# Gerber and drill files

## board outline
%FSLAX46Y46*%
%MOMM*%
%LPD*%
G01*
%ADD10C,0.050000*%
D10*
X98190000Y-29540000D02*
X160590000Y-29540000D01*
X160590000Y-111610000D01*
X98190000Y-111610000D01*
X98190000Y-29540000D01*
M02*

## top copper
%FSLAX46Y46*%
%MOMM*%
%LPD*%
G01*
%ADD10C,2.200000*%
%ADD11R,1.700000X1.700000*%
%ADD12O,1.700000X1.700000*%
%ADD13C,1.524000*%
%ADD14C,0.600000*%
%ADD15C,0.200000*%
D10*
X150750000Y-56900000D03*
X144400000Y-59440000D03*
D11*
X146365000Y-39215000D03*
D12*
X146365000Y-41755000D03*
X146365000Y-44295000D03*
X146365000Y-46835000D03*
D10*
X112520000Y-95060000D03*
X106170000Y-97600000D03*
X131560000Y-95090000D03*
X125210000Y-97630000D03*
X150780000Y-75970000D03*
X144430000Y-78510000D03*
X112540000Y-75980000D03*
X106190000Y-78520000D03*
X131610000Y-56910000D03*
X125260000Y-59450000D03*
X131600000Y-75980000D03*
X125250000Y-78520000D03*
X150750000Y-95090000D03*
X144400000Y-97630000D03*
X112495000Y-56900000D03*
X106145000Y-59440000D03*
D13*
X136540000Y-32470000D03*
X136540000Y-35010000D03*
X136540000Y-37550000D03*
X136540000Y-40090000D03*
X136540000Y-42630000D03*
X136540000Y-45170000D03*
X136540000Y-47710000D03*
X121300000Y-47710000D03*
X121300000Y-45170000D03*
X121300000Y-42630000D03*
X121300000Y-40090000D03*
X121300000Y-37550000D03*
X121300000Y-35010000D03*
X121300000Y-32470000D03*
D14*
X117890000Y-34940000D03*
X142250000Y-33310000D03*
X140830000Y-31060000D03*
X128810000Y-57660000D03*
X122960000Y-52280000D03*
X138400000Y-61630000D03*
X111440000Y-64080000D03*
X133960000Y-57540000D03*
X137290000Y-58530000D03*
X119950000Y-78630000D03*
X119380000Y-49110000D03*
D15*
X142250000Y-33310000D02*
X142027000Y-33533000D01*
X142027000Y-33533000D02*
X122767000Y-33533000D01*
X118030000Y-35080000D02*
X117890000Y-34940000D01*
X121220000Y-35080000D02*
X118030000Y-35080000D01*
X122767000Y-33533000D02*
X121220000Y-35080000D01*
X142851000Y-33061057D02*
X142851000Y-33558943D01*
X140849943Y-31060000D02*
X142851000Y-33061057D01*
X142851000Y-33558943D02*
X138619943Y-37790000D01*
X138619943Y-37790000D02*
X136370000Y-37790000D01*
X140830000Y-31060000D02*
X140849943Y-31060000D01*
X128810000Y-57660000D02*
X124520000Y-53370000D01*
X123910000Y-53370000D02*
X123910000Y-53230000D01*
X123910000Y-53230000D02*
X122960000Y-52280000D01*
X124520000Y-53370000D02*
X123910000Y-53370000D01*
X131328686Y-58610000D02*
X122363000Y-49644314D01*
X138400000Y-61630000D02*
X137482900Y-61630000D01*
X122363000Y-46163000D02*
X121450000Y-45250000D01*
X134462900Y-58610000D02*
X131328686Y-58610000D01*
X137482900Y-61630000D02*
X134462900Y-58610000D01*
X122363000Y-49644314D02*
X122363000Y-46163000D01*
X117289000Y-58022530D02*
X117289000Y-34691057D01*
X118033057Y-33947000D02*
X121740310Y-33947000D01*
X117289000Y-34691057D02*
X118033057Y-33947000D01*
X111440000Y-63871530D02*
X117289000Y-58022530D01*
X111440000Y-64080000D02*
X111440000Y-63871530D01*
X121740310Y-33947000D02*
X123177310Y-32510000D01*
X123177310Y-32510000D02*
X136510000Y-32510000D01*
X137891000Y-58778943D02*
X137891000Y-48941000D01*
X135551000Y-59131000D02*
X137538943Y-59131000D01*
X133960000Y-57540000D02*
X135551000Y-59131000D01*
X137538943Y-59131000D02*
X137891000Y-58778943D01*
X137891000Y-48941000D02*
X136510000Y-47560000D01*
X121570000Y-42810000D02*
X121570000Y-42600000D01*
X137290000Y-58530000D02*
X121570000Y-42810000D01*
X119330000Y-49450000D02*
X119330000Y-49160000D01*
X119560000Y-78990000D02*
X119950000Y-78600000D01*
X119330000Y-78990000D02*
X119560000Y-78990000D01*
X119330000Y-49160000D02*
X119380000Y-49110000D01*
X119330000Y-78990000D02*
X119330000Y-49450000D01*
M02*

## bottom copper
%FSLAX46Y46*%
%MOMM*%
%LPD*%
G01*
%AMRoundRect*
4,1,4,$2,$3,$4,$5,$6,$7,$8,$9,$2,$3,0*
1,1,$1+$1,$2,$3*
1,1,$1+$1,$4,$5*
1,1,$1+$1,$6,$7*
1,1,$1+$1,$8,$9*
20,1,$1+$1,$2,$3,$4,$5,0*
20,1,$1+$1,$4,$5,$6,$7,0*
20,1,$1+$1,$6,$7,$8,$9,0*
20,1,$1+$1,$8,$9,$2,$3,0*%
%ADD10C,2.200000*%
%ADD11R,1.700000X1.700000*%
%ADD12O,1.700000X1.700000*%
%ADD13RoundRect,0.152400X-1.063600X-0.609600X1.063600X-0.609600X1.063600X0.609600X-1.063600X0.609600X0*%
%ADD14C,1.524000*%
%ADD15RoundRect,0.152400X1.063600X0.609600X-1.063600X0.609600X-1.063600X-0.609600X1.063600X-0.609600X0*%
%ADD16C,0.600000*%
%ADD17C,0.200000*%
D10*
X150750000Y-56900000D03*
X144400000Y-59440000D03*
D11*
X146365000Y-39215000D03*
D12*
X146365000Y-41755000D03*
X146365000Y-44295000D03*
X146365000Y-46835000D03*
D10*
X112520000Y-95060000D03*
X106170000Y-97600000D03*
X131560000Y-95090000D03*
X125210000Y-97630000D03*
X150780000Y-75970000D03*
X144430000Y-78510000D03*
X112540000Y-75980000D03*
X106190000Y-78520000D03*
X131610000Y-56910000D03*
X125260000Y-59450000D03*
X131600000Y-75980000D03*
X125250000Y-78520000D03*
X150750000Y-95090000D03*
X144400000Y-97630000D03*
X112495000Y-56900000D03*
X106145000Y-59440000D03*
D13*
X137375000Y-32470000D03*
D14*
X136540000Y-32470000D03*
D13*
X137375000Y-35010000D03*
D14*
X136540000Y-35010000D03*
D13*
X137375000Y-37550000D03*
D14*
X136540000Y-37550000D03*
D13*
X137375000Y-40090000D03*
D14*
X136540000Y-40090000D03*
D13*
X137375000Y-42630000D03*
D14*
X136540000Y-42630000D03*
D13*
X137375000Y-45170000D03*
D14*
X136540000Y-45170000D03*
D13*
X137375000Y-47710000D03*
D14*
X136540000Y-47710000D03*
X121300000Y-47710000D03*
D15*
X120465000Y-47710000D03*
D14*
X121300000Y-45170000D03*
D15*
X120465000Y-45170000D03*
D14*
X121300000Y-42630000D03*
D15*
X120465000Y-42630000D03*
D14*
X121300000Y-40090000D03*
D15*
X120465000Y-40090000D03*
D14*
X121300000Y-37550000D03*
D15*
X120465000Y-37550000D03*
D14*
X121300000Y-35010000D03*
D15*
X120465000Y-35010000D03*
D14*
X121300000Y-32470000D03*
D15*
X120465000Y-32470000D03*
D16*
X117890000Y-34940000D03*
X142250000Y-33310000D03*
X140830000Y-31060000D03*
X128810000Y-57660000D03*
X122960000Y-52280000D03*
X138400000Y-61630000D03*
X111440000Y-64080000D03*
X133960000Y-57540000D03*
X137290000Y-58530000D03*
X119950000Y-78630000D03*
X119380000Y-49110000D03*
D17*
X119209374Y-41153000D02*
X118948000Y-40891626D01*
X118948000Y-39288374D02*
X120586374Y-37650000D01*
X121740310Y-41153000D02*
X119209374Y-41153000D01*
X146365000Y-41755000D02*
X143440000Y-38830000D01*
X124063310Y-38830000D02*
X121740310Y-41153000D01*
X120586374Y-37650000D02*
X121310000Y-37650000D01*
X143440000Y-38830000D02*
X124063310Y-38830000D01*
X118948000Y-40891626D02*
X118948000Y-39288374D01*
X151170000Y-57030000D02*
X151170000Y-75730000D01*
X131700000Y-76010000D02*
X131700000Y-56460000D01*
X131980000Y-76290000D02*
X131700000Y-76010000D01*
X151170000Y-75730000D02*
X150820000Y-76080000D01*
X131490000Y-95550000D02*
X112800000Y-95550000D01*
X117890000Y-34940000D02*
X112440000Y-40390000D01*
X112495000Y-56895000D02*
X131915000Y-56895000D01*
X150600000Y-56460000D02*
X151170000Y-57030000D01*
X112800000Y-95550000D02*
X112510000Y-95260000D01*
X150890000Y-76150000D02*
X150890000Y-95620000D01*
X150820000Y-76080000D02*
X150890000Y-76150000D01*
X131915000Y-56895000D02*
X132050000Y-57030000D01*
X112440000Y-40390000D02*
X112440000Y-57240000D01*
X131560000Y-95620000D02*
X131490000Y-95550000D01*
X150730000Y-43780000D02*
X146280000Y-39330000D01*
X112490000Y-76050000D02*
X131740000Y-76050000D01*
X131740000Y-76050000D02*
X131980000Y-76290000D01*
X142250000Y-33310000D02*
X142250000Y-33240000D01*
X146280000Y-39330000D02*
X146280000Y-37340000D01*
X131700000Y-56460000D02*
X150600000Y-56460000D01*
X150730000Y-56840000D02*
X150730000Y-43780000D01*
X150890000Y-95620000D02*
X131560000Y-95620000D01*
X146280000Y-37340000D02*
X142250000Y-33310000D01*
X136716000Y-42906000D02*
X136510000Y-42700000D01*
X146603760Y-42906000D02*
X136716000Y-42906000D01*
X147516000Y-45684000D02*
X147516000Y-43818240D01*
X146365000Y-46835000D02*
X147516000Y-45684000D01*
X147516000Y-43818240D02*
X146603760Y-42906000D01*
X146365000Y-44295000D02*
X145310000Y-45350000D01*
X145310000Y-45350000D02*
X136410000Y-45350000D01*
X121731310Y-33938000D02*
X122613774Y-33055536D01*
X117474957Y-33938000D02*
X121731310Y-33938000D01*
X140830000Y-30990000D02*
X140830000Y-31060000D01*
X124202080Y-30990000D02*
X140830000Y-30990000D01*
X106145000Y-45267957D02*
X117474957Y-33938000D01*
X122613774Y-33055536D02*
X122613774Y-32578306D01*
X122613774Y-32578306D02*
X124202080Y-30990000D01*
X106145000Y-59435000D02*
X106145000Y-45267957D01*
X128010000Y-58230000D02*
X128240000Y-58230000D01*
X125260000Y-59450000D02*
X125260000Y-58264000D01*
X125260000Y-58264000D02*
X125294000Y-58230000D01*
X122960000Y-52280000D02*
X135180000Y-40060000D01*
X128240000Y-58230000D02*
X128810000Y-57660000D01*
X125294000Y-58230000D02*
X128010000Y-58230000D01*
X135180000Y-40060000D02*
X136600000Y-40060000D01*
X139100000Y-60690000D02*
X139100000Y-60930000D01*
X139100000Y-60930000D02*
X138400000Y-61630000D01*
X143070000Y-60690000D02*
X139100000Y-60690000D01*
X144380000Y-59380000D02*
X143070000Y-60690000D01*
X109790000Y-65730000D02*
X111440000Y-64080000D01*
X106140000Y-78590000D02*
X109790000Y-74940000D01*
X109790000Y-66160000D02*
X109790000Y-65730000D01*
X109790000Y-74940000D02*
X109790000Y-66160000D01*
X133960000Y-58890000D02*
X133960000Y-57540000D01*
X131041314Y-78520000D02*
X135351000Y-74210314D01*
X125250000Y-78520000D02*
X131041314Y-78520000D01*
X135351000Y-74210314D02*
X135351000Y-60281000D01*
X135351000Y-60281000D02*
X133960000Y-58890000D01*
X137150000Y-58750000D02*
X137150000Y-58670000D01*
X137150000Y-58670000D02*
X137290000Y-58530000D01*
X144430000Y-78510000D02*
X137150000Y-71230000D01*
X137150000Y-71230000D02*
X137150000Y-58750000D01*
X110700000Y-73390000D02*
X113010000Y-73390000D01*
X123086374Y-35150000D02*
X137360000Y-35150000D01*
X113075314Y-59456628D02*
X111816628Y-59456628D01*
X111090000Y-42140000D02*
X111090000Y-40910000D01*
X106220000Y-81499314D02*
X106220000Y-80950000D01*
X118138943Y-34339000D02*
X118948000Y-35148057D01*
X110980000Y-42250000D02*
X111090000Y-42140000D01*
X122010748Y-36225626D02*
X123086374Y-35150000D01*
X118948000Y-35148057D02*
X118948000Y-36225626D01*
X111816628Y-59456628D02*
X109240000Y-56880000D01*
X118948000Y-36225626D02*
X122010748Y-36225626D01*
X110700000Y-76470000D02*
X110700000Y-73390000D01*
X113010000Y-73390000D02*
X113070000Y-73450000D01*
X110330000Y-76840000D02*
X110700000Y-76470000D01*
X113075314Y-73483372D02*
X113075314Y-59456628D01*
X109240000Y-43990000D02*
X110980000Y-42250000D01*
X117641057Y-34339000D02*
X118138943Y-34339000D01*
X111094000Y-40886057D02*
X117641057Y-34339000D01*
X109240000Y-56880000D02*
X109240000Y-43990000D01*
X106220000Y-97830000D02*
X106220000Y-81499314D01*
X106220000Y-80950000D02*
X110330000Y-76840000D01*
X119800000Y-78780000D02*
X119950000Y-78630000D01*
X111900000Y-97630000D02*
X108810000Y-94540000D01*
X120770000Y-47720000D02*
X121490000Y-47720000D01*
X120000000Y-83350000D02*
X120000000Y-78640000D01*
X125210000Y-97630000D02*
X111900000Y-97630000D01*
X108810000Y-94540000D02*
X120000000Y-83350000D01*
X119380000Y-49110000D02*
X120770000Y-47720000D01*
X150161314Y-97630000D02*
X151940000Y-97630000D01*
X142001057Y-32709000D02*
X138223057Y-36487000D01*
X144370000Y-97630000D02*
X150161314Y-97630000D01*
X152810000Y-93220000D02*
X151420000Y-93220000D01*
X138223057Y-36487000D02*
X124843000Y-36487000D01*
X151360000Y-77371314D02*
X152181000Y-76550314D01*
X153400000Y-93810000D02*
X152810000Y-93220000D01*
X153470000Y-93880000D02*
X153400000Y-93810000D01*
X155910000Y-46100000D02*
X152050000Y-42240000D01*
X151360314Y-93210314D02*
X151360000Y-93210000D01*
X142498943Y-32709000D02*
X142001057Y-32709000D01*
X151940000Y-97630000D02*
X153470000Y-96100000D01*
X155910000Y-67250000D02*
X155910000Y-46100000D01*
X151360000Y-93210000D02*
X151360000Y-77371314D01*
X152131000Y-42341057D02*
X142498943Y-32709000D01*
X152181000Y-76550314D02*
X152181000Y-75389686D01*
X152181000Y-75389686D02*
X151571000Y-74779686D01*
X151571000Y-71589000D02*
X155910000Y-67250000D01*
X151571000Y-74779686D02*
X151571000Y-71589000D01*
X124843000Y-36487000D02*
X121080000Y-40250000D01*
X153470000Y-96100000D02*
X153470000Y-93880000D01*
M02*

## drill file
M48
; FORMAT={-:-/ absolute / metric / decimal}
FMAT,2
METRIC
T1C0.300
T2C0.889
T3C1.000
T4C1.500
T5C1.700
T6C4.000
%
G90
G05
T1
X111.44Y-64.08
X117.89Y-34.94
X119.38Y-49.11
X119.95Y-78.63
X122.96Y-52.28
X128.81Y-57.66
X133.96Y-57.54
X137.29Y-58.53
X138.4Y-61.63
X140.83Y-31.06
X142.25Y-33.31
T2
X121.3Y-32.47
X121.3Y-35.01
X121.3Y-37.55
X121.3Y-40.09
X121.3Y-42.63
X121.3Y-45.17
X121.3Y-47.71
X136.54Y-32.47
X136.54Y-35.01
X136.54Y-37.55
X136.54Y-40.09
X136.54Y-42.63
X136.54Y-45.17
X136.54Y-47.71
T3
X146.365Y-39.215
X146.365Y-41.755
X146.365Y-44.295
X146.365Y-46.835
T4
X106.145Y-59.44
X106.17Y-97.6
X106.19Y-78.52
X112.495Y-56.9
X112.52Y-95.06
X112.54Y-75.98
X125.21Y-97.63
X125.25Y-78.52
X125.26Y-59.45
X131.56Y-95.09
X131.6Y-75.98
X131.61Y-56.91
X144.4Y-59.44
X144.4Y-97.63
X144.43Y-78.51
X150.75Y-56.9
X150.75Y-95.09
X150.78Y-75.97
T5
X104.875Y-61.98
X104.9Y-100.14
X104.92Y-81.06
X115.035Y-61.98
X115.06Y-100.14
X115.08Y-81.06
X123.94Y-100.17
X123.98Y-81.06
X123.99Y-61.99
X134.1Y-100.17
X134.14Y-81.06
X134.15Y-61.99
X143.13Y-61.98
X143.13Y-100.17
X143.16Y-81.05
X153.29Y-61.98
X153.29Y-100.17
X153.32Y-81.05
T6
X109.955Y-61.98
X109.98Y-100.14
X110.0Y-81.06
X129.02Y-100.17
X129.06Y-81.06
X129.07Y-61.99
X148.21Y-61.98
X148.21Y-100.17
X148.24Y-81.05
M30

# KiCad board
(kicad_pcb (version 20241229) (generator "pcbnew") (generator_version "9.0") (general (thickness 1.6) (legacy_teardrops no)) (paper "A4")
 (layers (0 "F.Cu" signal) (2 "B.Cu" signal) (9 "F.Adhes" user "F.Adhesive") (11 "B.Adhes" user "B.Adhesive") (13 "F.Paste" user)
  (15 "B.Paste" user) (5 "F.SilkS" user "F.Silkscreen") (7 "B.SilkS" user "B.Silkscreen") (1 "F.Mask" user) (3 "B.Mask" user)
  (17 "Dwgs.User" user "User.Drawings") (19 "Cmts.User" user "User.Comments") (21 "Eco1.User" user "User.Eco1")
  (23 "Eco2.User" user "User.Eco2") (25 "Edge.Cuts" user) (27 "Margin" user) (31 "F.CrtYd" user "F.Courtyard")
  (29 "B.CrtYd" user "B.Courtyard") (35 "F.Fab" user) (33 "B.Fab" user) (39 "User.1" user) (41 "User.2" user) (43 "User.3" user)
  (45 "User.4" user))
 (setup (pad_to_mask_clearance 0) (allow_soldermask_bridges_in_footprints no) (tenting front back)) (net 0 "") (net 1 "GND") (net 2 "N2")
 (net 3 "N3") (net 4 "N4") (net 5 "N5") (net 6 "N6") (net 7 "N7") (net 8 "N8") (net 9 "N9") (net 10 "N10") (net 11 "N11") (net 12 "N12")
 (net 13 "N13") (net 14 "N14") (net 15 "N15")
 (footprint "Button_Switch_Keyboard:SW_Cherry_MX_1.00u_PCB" (layer "F.Cu") (at 150.75 56.9)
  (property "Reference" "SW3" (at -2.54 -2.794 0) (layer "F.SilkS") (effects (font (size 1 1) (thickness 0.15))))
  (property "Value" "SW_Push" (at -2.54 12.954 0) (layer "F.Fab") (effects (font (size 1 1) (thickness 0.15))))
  (pad "" np_thru_hole circle (at -7.62 5.08) (size 1.7 1.7) (drill 1.7) (layers "*.Cu" "*.Mask"))
  (pad "" np_thru_hole circle (at -2.54 5.08) (size 4 4) (drill 4) (layers "*.Cu" "*.Mask"))
  (pad "" np_thru_hole circle (at 2.54 5.08) (size 1.7 1.7) (drill 1.7) (layers "*.Cu" "*.Mask"))
  (pad "1" thru_hole circle (at 0 0) (size 2.2 2.2) (drill 1.5) (layers "*.Cu" "*.Mask") (remove_unused_layers no) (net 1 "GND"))
  (pad "2" thru_hole circle (at -6.35 2.54) (size 2.2 2.2) (drill 1.5) (layers "*.Cu" "*.Mask") (remove_unused_layers no) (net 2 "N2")))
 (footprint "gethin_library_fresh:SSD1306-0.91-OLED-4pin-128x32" (layer "F.Cu") (at 109.865 37.025)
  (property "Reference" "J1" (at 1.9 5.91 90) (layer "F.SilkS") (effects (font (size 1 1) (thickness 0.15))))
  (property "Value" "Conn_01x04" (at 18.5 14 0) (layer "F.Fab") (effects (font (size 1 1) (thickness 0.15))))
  (pad "1" thru_hole rect (at 36.5 2.19) (size 1.7 1.7) (drill 1) (layers "*.Cu" "*.Mask") (remove_unused_layers no) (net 1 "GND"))
  (pad "2" thru_hole oval (at 36.5 4.73) (size 1.7 1.7) (drill 1) (layers "*.Cu" "*.Mask") (remove_unused_layers no) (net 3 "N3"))
  (pad "3" thru_hole oval (at 36.5 7.27) (size 1.7 1.7) (drill 1) (layers "*.Cu" "*.Mask") (remove_unused_layers no) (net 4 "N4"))
  (pad "4" thru_hole oval (at 36.5 9.81) (size 1.7 1.7) (drill 1) (layers "*.Cu" "*.Mask") (remove_unused_layers no) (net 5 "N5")))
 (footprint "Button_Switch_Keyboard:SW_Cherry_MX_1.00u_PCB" (layer "F.Cu") (at 112.52 95.06)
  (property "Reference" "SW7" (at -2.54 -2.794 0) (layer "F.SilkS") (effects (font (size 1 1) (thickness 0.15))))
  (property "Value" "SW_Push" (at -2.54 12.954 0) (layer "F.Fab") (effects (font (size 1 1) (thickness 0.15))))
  (pad "" np_thru_hole circle (at -7.62 5.08) (size 1.7 1.7) (drill 1.7) (layers "*.Cu" "*.Mask"))
  (pad "" np_thru_hole circle (at -2.54 5.08) (size 4 4) (drill 4) (layers "*.Cu" "*.Mask"))
  (pad "" np_thru_hole circle (at 2.54 5.08) (size 1.7 1.7) (drill 1.7) (layers "*.Cu" "*.Mask"))
  (pad "1" thru_hole circle (at 0 0) (size 2.2 2.2) (drill 1.5) (layers "*.Cu" "*.Mask") (remove_unused_layers no) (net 1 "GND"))
  (pad "2" thru_hole circle (at -6.35 2.54) (size 2.2 2.2) (drill 1.5) (layers "*.Cu" "*.Mask") (remove_unused_layers no) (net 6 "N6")))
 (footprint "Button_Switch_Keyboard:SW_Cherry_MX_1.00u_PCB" (layer "F.Cu") (at 131.56 95.09)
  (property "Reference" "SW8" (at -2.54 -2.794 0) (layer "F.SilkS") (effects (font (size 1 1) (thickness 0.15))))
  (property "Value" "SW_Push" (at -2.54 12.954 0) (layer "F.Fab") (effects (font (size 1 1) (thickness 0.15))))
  (pad "" np_thru_hole circle (at -7.62 5.08) (size 1.7 1.7) (drill 1.7) (layers "*.Cu" "*.Mask"))
  (pad "" np_thru_hole circle (at -2.54 5.08) (size 4 4) (drill 4) (layers "*.Cu" "*.Mask"))
  (pad "" np_thru_hole circle (at 2.54 5.08) (size 1.7 1.7) (drill 1.7) (layers "*.Cu" "*.Mask"))
  (pad "1" thru_hole circle (at 0 0) (size 2.2 2.2) (drill 1.5) (layers "*.Cu" "*.Mask") (remove_unused_layers no) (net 1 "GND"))
  (pad "2" thru_hole circle (at -6.35 2.54) (size 2.2 2.2) (drill 1.5) (layers "*.Cu" "*.Mask") (remove_unused_layers no) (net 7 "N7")))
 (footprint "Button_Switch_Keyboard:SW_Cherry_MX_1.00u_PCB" (layer "F.Cu") (at 150.78 75.97)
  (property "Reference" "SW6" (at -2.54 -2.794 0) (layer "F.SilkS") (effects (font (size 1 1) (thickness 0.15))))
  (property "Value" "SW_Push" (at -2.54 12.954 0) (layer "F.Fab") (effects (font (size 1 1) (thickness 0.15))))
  (pad "" np_thru_hole circle (at -7.62 5.08) (size 1.7 1.7) (drill 1.7) (layers "*.Cu" "*.Mask"))
  (pad "" np_thru_hole circle (at -2.54 5.08) (size 4 4) (drill 4) (layers "*.Cu" "*.Mask"))
  (pad "" np_thru_hole circle (at 2.54 5.08) (size 1.7 1.7) (drill 1.7) (layers "*.Cu" "*.Mask"))
  (pad "1" thru_hole circle (at 0 0) (size 2.2 2.2) (drill 1.5) (layers "*.Cu" "*.Mask") (remove_unused_layers no) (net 1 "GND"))
  (pad "2" thru_hole circle (at -6.35 2.54) (size 2.2 2.2) (drill 1.5) (layers "*.Cu" "*.Mask") (remove_unused_layers no) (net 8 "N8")))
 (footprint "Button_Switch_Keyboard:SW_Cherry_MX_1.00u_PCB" (layer "F.Cu") (at 112.54 75.98)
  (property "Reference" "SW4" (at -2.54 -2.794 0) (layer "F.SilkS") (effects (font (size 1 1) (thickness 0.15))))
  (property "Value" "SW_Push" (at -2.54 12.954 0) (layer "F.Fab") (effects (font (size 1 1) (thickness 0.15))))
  (pad "" np_thru_hole circle (at -7.62 5.08) (size 1.7 1.7) (drill 1.7) (layers "*.Cu" "*.Mask"))
  (pad "" np_thru_hole circle (at -2.54 5.08) (size 4 4) (drill 4) (layers "*.Cu" "*.Mask"))
  (pad "" np_thru_hole circle (at 2.54 5.08) (size 1.7 1.7) (drill 1.7) (layers "*.Cu" "*.Mask"))
  (pad "1" thru_hole circle (at 0 0) (size 2.2 2.2) (drill 1.5) (layers "*.Cu" "*.Mask") (remove_unused_layers no) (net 1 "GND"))
  (pad "2" thru_hole circle (at -6.35 2.54) (size 2.2 2.2) (drill 1.5) (layers "*.Cu" "*.Mask") (remove_unused_layers no) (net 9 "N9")))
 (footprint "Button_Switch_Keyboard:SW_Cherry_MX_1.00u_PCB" (layer "F.Cu") (at 131.61 56.91)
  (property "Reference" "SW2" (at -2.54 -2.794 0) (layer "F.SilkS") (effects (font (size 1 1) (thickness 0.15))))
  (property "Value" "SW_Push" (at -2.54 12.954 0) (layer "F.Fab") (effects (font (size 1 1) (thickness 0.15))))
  (pad "" np_thru_hole circle (at -7.62 5.08) (size 1.7 1.7) (drill 1.7) (layers "*.Cu" "*.Mask"))
  (pad "" np_thru_hole circle (at -2.54 5.08) (size 4 4) (drill 4) (layers "*.Cu" "*.Mask"))
  (pad "" np_thru_hole circle (at 2.54 5.08) (size 1.7 1.7) (drill 1.7) (layers "*.Cu" "*.Mask"))
  (pad "1" thru_hole circle (at 0 0) (size 2.2 2.2) (drill 1.5) (layers "*.Cu" "*.Mask") (remove_unused_layers no) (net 1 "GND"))
  (pad "2" thru_hole circle (at -6.35 2.54) (size 2.2 2.2) (drill 1.5) (layers "*.Cu" "*.Mask") (remove_unused_layers no) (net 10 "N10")))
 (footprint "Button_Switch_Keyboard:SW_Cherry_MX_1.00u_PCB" (layer "F.Cu") (at 131.6 75.98)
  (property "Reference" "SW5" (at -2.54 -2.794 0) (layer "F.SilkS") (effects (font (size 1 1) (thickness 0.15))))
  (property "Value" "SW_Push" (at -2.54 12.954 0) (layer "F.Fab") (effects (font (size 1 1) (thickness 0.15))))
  (pad "" np_thru_hole circle (at -7.62 5.08) (size 1.7 1.7) (drill 1.7) (layers "*.Cu" "*.Mask"))
  (pad "" np_thru_hole circle (at -2.54 5.08) (size 4 4) (drill 4) (layers "*.Cu" "*.Mask"))
  (pad "" np_thru_hole circle (at 2.54 5.08) (size 1.7 1.7) (drill 1.7) (layers "*.Cu" "*.Mask"))
  (pad "1" thru_hole circle (at 0 0) (size 2.2 2.2) (drill 1.5) (layers "*.Cu" "*.Mask") (remove_unused_layers no) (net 1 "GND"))
  (pad "2" thru_hole circle (at -6.35 2.54) (size 2.2 2.2) (drill 1.5) (layers "*.Cu" "*.Mask") (remove_unused_layers no) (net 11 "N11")))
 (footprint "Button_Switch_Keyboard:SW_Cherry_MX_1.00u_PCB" (layer "F.Cu") (at 150.75 95.09)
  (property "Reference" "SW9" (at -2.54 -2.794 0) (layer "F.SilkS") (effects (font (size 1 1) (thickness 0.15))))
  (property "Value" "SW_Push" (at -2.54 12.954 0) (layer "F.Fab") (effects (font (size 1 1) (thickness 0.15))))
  (pad "" np_thru_hole circle (at -7.62 5.08) (size 1.7 1.7) (drill 1.7) (layers "*.Cu" "*.Mask"))
  (pad "" np_thru_hole circle (at -2.54 5.08) (size 4 4) (drill 4) (layers "*.Cu" "*.Mask"))
  (pad "" np_thru_hole circle (at 2.54 5.08) (size 1.7 1.7) (drill 1.7) (layers "*.Cu" "*.Mask"))
  (pad "1" thru_hole circle (at 0 0) (size 2.2 2.2) (drill 1.5) (layers "*.Cu" "*.Mask") (remove_unused_layers no) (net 1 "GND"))
  (pad "2" thru_hole circle (at -6.35 2.54) (size 2.2 2.2) (drill 1.5) (layers "*.Cu" "*.Mask") (remove_unused_layers no) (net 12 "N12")))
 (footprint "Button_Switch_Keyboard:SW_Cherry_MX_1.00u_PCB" (layer "F.Cu") (at 112.495 56.9)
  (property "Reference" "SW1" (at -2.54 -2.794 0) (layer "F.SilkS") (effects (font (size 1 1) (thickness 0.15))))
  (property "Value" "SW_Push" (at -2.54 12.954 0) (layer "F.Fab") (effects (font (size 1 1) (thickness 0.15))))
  (pad "" np_thru_hole circle (at -7.62 5.08) (size 1.7 1.7) (drill 1.7) (layers "*.Cu" "*.Mask"))
  (pad "" np_thru_hole circle (at -2.54 5.08) (size 4 4) (drill 4) (layers "*.Cu" "*.Mask"))
  (pad "" np_thru_hole circle (at 2.54 5.08) (size 1.7 1.7) (drill 1.7) (layers "*.Cu" "*.Mask"))
  (pad "1" thru_hole circle (at 0 0) (size 2.2 2.2) (drill 1.5) (layers "*.Cu" "*.Mask") (remove_unused_layers no) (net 1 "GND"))
  (pad "2" thru_hole circle (at -6.35 2.54) (size 2.2 2.2) (drill 1.5) (layers "*.Cu" "*.Mask") (remove_unused_layers no) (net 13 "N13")))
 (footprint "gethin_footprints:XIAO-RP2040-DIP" (layer "B.Cu") (at 128.92 40.09 180)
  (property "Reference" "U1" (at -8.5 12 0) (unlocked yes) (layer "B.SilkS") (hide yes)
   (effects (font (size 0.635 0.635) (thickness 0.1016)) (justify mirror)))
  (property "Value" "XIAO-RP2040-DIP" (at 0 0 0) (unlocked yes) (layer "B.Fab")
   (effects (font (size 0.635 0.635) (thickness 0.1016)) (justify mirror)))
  (pad "1" smd roundrect (at -8.455 7.62) (size 2.432 1.524) (layers "B.Cu" "B.Mask") (roundrect_rratio 0.1) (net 9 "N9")
   (thermal_bridge_angle 45))
  (pad "1" thru_hole circle (at -7.62 7.62) (size 1.524 1.524) (drill 0.889) (layers "*.Cu" "*.Mask") (remove_unused_layers no) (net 9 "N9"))
  (pad "2" smd roundrect (at -8.455 5.08) (size 2.432 1.524) (layers "B.Cu" "B.Mask") (roundrect_rratio 0.1) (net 6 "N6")
   (thermal_bridge_angle 45))
  (pad "2" thru_hole circle (at -7.62 5.08) (size 1.524 1.524) (drill 0.889) (layers "*.Cu" "*.Mask") (remove_unused_layers no) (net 6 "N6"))
  (pad "3" smd roundrect (at -8.455 2.54) (size 2.432 1.524) (layers "B.Cu" "B.Mask") (roundrect_rratio 0.1) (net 13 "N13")
   (thermal_bridge_angle 45))
  (pad "3" thru_hole circle (at -7.62 2.54) (size 1.524 1.524) (drill 0.889) (layers "*.Cu" "*.Mask") (remove_unused_layers no)
   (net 13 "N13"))
  (pad "4" smd roundrect (at -8.455 0) (size 2.432 1.524) (layers "B.Cu" "B.Mask") (roundrect_rratio 0.1) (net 10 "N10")
   (thermal_bridge_angle 45))
  (pad "4" thru_hole circle (at -7.62 0) (size 1.524 1.524) (drill 0.889) (layers "*.Cu" "*.Mask") (remove_unused_layers no) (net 10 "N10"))
  (pad "5" smd roundrect (at -8.455 -2.54) (size 2.432 1.524) (layers "B.Cu" "B.Mask") (roundrect_rratio 0.1) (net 5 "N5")
   (thermal_bridge_angle 45))
  (pad "5" thru_hole circle (at -7.62 -2.54) (size 1.524 1.524) (drill 0.889) (layers "*.Cu" "*.Mask") (remove_unused_layers no)
   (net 5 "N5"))
  (pad "6" smd roundrect (at -8.455 -5.08) (size 2.432 1.524) (layers "B.Cu" "B.Mask") (roundrect_rratio 0.1) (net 4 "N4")
   (thermal_bridge_angle 45))
  (pad "6" thru_hole circle (at -7.62 -5.08) (size 1.524 1.524) (drill 0.889) (layers "*.Cu" "*.Mask") (remove_unused_layers no)
   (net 4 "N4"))
  (pad "7" smd roundrect (at -8.455 -7.62) (size 2.432 1.524) (layers "B.Cu" "B.Mask") (roundrect_rratio 0.1) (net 11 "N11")
   (thermal_bridge_angle 45))
  (pad "7" thru_hole circle (at -7.62 -7.62) (size 1.524 1.524) (drill 0.889) (layers "*.Cu" "*.Mask") (remove_unused_layers no)
   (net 11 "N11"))
  (pad "8" thru_hole circle (at 7.62 -7.62 180) (size 1.524 1.524) (drill 0.889) (layers "*.Cu" "*.Mask") (remove_unused_layers no)
   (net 7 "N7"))
  (pad "8" smd roundrect (at 8.455 -7.62 180) (size 2.432 1.524) (layers "B.Cu" "B.Mask") (roundrect_rratio 0.1) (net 7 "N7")
   (thermal_bridge_angle 45))
  (pad "9" thru_hole circle (at 7.62 -5.08 180) (size 1.524 1.524) (drill 0.889) (layers "*.Cu" "*.Mask") (remove_unused_layers no)
   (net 2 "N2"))
  (pad "9" smd roundrect (at 8.455 -5.08 180) (size 2.432 1.524) (layers "B.Cu" "B.Mask") (roundrect_rratio 0.1) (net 2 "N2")
   (thermal_bridge_angle 45))
  (pad "10" thru_hole circle (at 7.62 -2.54 180) (size 1.524 1.524) (drill 0.889) (layers "*.Cu" "*.Mask") (remove_unused_layers no)
   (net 8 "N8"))
  (pad "10" smd roundrect (at 8.455 -2.54 180) (size 2.432 1.524) (layers "B.Cu" "B.Mask") (roundrect_rratio 0.1) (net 8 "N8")
   (thermal_bridge_angle 45))
  (pad "11" thru_hole circle (at 7.62 0 180) (size 1.524 1.524) (drill 0.889) (layers "*.Cu" "*.Mask") (remove_unused_layers no)
   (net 12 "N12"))
  (pad "11" smd roundrect (at 8.455 0 180) (size 2.432 1.524) (layers "B.Cu" "B.Mask") (roundrect_rratio 0.1) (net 12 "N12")
   (thermal_bridge_angle 45))
  (pad "12" thru_hole circle (at 7.62 2.54 180) (size 1.524 1.524) (drill 0.889) (layers "*.Cu" "*.Mask") (remove_unused_layers no)
   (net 3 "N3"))
  (pad "12" smd roundrect (at 8.455 2.54 180) (size 2.432 1.524) (layers "B.Cu" "B.Mask") (roundrect_rratio 0.1) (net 3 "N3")
   (thermal_bridge_angle 45))
  (pad "13" thru_hole circle (at 7.62 5.08 180) (size 1.524 1.524) (drill 0.889) (layers "*.Cu" "*.Mask") (remove_unused_layers no)
   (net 1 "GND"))
  (pad "13" smd roundrect (at 8.455 5.08 180) (size 2.432 1.524) (layers "B.Cu" "B.Mask") (roundrect_rratio 0.1) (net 1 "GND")
   (thermal_bridge_angle 45))
  (pad "14" thru_hole circle (at 7.62 7.62 180) (size 1.524 1.524) (drill 0.889) (layers "*.Cu" "*.Mask") (remove_unused_layers no)
   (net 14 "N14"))
  (pad "14" smd roundrect (at 8.455 7.62 180) (size 2.432 1.524) (layers "B.Cu" "B.Mask") (roundrect_rratio 0.1) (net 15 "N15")
   (thermal_bridge_angle 45)))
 (gr_rect (start 98.19 29.54) (end 160.59 111.61) (stroke (width 0.05) (type default)) (fill no) (layer "Edge.Cuts"))
 (segment (start 119.209374 41.153) (end 118.948 40.891626) (width 0.2) (layer "B.Cu") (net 3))
 (segment (start 118.948 39.288374) (end 120.586374 37.65) (width 0.2) (layer "B.Cu") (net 3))
 (segment (start 121.74031 41.153) (end 119.209374 41.153) (width 0.2) (layer "B.Cu") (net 3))
 (segment (start 146.365 41.755) (end 143.44 38.83) (width 0.2) (layer "B.Cu") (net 3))
 (segment (start 124.06331 38.83) (end 121.74031 41.153) (width 0.2) (layer "B.Cu") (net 3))
 (segment (start 120.586374 37.65) (end 121.31 37.65) (width 0.2) (layer "B.Cu") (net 3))
 (segment (start 143.44 38.83) (end 124.06331 38.83) (width 0.2) (layer "B.Cu") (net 3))
 (segment (start 118.948 40.891626) (end 118.948 39.288374) (width 0.2) (layer "B.Cu") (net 3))
 (segment (start 142.25 33.31) (end 142.027 33.533) (width 0.2) (layer "F.Cu") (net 1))
 (segment (start 142.027 33.533) (end 122.767 33.533) (width 0.2) (layer "F.Cu") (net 1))
 (segment (start 118.03 35.08) (end 117.89 34.94) (width 0.2) (layer "F.Cu") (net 1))
 (segment (start 121.22 35.08) (end 118.03 35.08) (width 0.2) (layer "F.Cu") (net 1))
 (segment (start 122.767 33.533) (end 121.22 35.08) (width 0.2) (layer "F.Cu") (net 1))
 (via (at 117.89 34.94) (size 0.6) (drill 0.3) (layers "F.Cu" "B.Cu") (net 1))
 (via (at 142.25 33.31) (size 0.6) (drill 0.3) (layers "F.Cu" "B.Cu") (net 1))
 (segment (start 151.17 57.03) (end 151.17 75.73) (width 0.2) (layer "B.Cu") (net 1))
 (segment (start 131.7 76.01) (end 131.7 56.46) (width 0.2) (layer "B.Cu") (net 1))
 (segment (start 131.98 76.29) (end 131.7 76.01) (width 0.2) (layer "B.Cu") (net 1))
 (segment (start 151.17 75.73) (end 150.82 76.08) (width 0.2) (layer "B.Cu") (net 1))
 (segment (start 131.49 95.55) (end 112.8 95.55) (width 0.2) (layer "B.Cu") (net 1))
 (segment (start 117.89 34.94) (end 112.44 40.39) (width 0.2) (layer "B.Cu") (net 1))
 (segment (start 112.495 56.895) (end 131.915 56.895) (width 0.2) (layer "B.Cu") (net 1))
 (segment (start 150.6 56.46) (end 151.17 57.03) (width 0.2) (layer "B.Cu") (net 1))
 (segment (start 112.8 95.55) (end 112.51 95.26) (width 0.2) (layer "B.Cu") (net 1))
 (segment (start 150.89 76.15) (end 150.89 95.62) (width 0.2) (layer "B.Cu") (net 1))
 (segment (start 150.82 76.08) (end 150.89 76.15) (width 0.2) (layer "B.Cu") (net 1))
 (segment (start 131.915 56.895) (end 132.05 57.03) (width 0.2) (layer "B.Cu") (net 1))
 (segment (start 112.44 40.39) (end 112.44 57.24) (width 0.2) (layer "B.Cu") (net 1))
 (segment (start 131.56 95.62) (end 131.49 95.55) (width 0.2) (layer "B.Cu") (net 1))
 (segment (start 150.73 43.78) (end 146.28 39.33) (width 0.2) (layer "B.Cu") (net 1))
 (segment (start 112.49 76.05) (end 131.74 76.05) (width 0.2) (layer "B.Cu") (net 1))
 (segment (start 131.74 76.05) (end 131.98 76.29) (width 0.2) (layer "B.Cu") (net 1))
 (segment (start 142.25 33.31) (end 142.25 33.24) (width 0.2) (layer "B.Cu") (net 1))
 (segment (start 146.28 39.33) (end 146.28 37.34) (width 0.2) (layer "B.Cu") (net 1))
 (segment (start 131.7 56.46) (end 150.6 56.46) (width 0.2) (layer "B.Cu") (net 1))
 (segment (start 150.73 56.84) (end 150.73 43.78) (width 0.2) (layer "B.Cu") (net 1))
 (segment (start 150.89 95.62) (end 131.56 95.62) (width 0.2) (layer "B.Cu") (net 1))
 (segment (start 146.28 37.34) (end 142.25 33.31) (width 0.2) (layer "B.Cu") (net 1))
 (segment (start 136.716 42.906) (end 136.51 42.7) (width 0.2) (layer "B.Cu") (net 5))
 (segment (start 146.60376 42.906) (end 136.716 42.906) (width 0.2) (layer "B.Cu") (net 5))
 (segment (start 147.516 45.684) (end 147.516 43.81824) (width 0.2) (layer "B.Cu") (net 5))
 (segment (start 146.365 46.835) (end 147.516 45.684) (width 0.2) (layer "B.Cu") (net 5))
 (segment (start 147.516 43.81824) (end 146.60376 42.906) (width 0.2) (layer "B.Cu") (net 5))
 (segment (start 146.365 44.295) (end 145.31 45.35) (width 0.2) (layer "B.Cu") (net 4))
 (segment (start 145.31 45.35) (end 136.41 45.35) (width 0.2) (layer "B.Cu") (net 4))
 (segment (start 142.851 33.061057) (end 142.851 33.558943) (width 0.2) (layer "F.Cu") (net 13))
 (segment (start 140.849943 31.06) (end 142.851 33.061057) (width 0.2) (layer "F.Cu") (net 13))
 (segment (start 142.851 33.558943) (end 138.619943 37.79) (width 0.2) (layer "F.Cu") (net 13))
 (segment (start 138.619943 37.79) (end 136.37 37.79) (width 0.2) (layer "F.Cu") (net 13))
 (segment (start 140.83 31.06) (end 140.849943 31.06) (width 0.2) (layer "F.Cu") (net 13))
 (via (at 140.83 31.06) (size 0.6) (drill 0.3) (layers "F.Cu" "B.Cu") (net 13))
 (segment (start 121.73131 33.938) (end 122.613774 33.055536) (width 0.2) (layer "B.Cu") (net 13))
 (segment (start 117.474957 33.938) (end 121.73131 33.938) (width 0.2) (layer "B.Cu") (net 13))
 (segment (start 140.83 30.99) (end 140.83 31.06) (width 0.2) (layer "B.Cu") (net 13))
 (segment (start 124.20208 30.99) (end 140.83 30.99) (width 0.2) (layer "B.Cu") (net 13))
 (segment (start 106.145 45.267957) (end 117.474957 33.938) (width 0.2) (layer "B.Cu") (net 13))
 (segment (start 122.613774 33.055536) (end 122.613774 32.578306) (width 0.2) (layer "B.Cu") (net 13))
 (segment (start 122.613774 32.578306) (end 124.20208 30.99) (width 0.2) (layer "B.Cu") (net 13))
 (segment (start 106.145 59.435) (end 106.145 45.267957) (width 0.2) (layer "B.Cu") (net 13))
 (segment (start 128.81 57.66) (end 124.52 53.37) (width 0.2) (layer "F.Cu") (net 10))
 (segment (start 123.91 53.37) (end 123.91 53.23) (width 0.2) (layer "F.Cu") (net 10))
 (segment (start 123.91 53.23) (end 122.96 52.28) (width 0.2) (layer "F.Cu") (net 10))
 (segment (start 124.52 53.37) (end 123.91 53.37) (width 0.2) (layer "F.Cu") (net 10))
 (via (at 128.81 57.66) (size 0.6) (drill 0.3) (layers "F.Cu" "B.Cu") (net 10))
 (via (at 122.96 52.28) (size 0.6) (drill 0.3) (layers "F.Cu" "B.Cu") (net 10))
 (segment (start 128.01 58.23) (end 128.24 58.23) (width 0.2) (layer "B.Cu") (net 10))
 (segment (start 125.26 59.45) (end 125.26 58.264) (width 0.2) (layer "B.Cu") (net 10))
 (segment (start 125.26 58.264) (end 125.294 58.23) (width 0.2) (layer "B.Cu") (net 10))
 (segment (start 122.96 52.28) (end 135.18 40.06) (width 0.2) (layer "B.Cu") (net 10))
 (segment (start 128.24 58.23) (end 128.81 57.66) (width 0.2) (layer "B.Cu") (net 10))
 (segment (start 125.294 58.23) (end 128.01 58.23) (width 0.2) (layer "B.Cu") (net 10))
 (segment (start 135.18 40.06) (end 136.6 40.06) (width 0.2) (layer "B.Cu") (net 10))
 (segment (start 131.328686 58.61) (end 122.363 49.644314) (width 0.2) (layer "F.Cu") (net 2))
 (segment (start 138.4 61.63) (end 137.4829 61.63) (width 0.2) (layer "F.Cu") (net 2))
 (segment (start 122.363 46.163) (end 121.45 45.25) (width 0.2) (layer "F.Cu") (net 2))
 (segment (start 134.4629 58.61) (end 131.328686 58.61) (width 0.2) (layer "F.Cu") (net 2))
 (segment (start 137.4829 61.63) (end 134.4629 58.61) (width 0.2) (layer "F.Cu") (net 2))
 (segment (start 122.363 49.644314) (end 122.363 46.163) (width 0.2) (layer "F.Cu") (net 2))
 (via (at 138.4 61.63) (size 0.6) (drill 0.3) (layers "F.Cu" "B.Cu") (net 2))
 (segment (start 139.1 60.69) (end 139.1 60.93) (width 0.2) (layer "B.Cu") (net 2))
 (segment (start 139.1 60.93) (end 138.4 61.63) (width 0.2) (layer "B.Cu") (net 2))
 (segment (start 143.07 60.69) (end 139.1 60.69) (width 0.2) (layer "B.Cu") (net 2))
 (segment (start 144.38 59.38) (end 143.07 60.69) (width 0.2) (layer "B.Cu") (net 2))
 (segment (start 117.289 58.02253) (end 117.289 34.691057) (width 0.2) (layer "F.Cu") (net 9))
 (segment (start 118.033057 33.947) (end 121.74031 33.947) (width 0.2) (layer "F.Cu") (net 9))
 (segment (start 117.289 34.691057) (end 118.033057 33.947) (width 0.2) (layer "F.Cu") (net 9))
 (segment (start 111.44 63.87153) (end 117.289 58.02253) (width 0.2) (layer "F.Cu") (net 9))
 (segment (start 111.44 64.08) (end 111.44 63.87153) (width 0.2) (layer "F.Cu") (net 9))
 (segment (start 121.74031 33.947) (end 123.17731 32.51) (width 0.2) (layer "F.Cu") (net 9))
 (segment (start 123.17731 32.51) (end 136.51 32.51) (width 0.2) (layer "F.Cu") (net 9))
 (via (at 111.44 64.08) (size 0.6) (drill 0.3) (layers "F.Cu" "B.Cu") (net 9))
 (segment (start 109.79 65.73) (end 111.44 64.08) (width 0.2) (layer "B.Cu") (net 9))
 (segment (start 106.14 78.59) (end 109.79 74.94) (width 0.2) (layer "B.Cu") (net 9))
 (segment (start 109.79 66.16) (end 109.79 65.73) (width 0.2) (layer "B.Cu") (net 9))
 (segment (start 109.79 74.94) (end 109.79 66.16) (width 0.2) (layer "B.Cu") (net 9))
 (segment (start 137.891 58.778943) (end 137.891 48.941) (width 0.2) (layer "F.Cu") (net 11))
 (segment (start 135.551 59.131) (end 137.538943 59.131) (width 0.2) (layer "F.Cu") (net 11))
 (segment (start 133.96 57.54) (end 135.551 59.131) (width 0.2) (layer "F.Cu") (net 11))
 (segment (start 137.538943 59.131) (end 137.891 58.778943) (width 0.2) (layer "F.Cu") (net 11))
 (segment (start 137.891 48.941) (end 136.51 47.56) (width 0.2) (layer "F.Cu") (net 11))
 (via (at 133.96 57.54) (size 0.6) (drill 0.3) (layers "F.Cu" "B.Cu") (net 11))
 (segment (start 133.96 58.89) (end 133.96 57.54) (width 0.2) (layer "B.Cu") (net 11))
 (segment (start 131.041314 78.52) (end 135.351 74.210314) (width 0.2) (layer "B.Cu") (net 11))
 (segment (start 125.25 78.52) (end 131.041314 78.52) (width 0.2) (layer "B.Cu") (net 11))
 (segment (start 135.351 74.210314) (end 135.351 60.281) (width 0.2) (layer "B.Cu") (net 11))
 (segment (start 135.351 60.281) (end 133.96 58.89) (width 0.2) (layer "B.Cu") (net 11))
 (segment (start 121.57 42.81) (end 121.57 42.6) (width 0.2) (layer "F.Cu") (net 8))
 (segment (start 137.29 58.53) (end 121.57 42.81) (width 0.2) (layer "F.Cu") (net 8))
 (via (at 137.29 58.53) (size 0.6) (drill 0.3) (layers "F.Cu" "B.Cu") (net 8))
 (segment (start 137.15 58.75) (end 137.15 58.67) (width 0.2) (layer "B.Cu") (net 8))
 (segment (start 137.15 58.67) (end 137.29 58.53) (width 0.2) (layer "B.Cu") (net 8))
 (segment (start 144.43 78.51) (end 137.15 71.23) (width 0.2) (layer "B.Cu") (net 8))
 (segment (start 137.15 71.23) (end 137.15 58.75) (width 0.2) (layer "B.Cu") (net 8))
 (segment (start 110.7 73.39) (end 113.01 73.39) (width 0.2) (layer "B.Cu") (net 6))
 (segment (start 123.086374 35.15) (end 137.36 35.15) (width 0.2) (layer "B.Cu") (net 6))
 (segment (start 113.075314 59.456628) (end 111.816628 59.456628) (width 0.2) (layer "B.Cu") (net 6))
 (segment (start 111.09 42.14) (end 111.09 40.91) (width 0.2) (layer "B.Cu") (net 6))
 (segment (start 106.22 81.499314) (end 106.22 80.95) (width 0.2) (layer "B.Cu") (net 6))
 (segment (start 118.138943 34.339) (end 118.948 35.148057) (width 0.2) (layer "B.Cu") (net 6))
 (segment (start 110.98 42.25) (end 111.09 42.14) (width 0.2) (layer "B.Cu") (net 6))
 (segment (start 122.010748 36.225626) (end 123.086374 35.15) (width 0.2) (layer "B.Cu") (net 6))
 (segment (start 118.948 35.148057) (end 118.948 36.225626) (width 0.2) (layer "B.Cu") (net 6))
 (segment (start 111.816628 59.456628) (end 109.24 56.88) (width 0.2) (layer "B.Cu") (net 6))
 (segment (start 118.948 36.225626) (end 122.010748 36.225626) (width 0.2) (layer "B.Cu") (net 6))
 (segment (start 110.7 76.47) (end 110.7 73.39) (width 0.2) (layer "B.Cu") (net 6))
 (segment (start 113.01 73.39) (end 113.07 73.45) (width 0.2) (layer "B.Cu") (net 6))
 (segment (start 110.33 76.84) (end 110.7 76.47) (width 0.2) (layer "B.Cu") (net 6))
 (segment (start 113.075314 73.483372) (end 113.075314 59.456628) (width 0.2) (layer "B.Cu") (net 6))
 (segment (start 109.24 43.99) (end 110.98 42.25) (width 0.2) (layer "B.Cu") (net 6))
 (segment (start 117.641057 34.339) (end 118.138943 34.339) (width 0.2) (layer "B.Cu") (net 6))
 (segment (start 111.094 40.886057) (end 117.641057 34.339) (width 0.2) (layer "B.Cu") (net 6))
 (segment (start 109.24 56.88) (end 109.24 43.99) (width 0.2) (layer "B.Cu") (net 6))
 (segment (start 106.22 97.83) (end 106.22 81.499314) (width 0.2) (layer "B.Cu") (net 6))
 (segment (start 106.22 80.95) (end 110.33 76.84) (width 0.2) (layer "B.Cu") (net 6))
 (segment (start 119.33 49.45) (end 119.33 49.16) (width 0.2) (layer "F.Cu") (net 7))
 (segment (start 119.56 78.99) (end 119.95 78.6) (width 0.2) (layer "F.Cu") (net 7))
 (segment (start 119.33 78.99) (end 119.56 78.99) (width 0.2) (layer "F.Cu") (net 7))
 (segment (start 119.33 49.16) (end 119.38 49.11) (width 0.2) (layer "F.Cu") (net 7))
 (segment (start 119.33 78.99) (end 119.33 49.45) (width 0.2) (layer "F.Cu") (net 7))
 (via (at 119.95 78.63) (size 0.6) (drill 0.3) (layers "F.Cu" "B.Cu") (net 7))
 (via (at 119.38 49.11) (size 0.6) (drill 0.3) (layers "F.Cu" "B.Cu") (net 7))
 (segment (start 119.8 78.78) (end 119.95 78.63) (width 0.2) (layer "B.Cu") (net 7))
 (segment (start 111.9 97.63) (end 108.81 94.54) (width 0.2) (layer "B.Cu") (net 7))
 (segment (start 120.77 47.72) (end 121.49 47.72) (width 0.2) (layer "B.Cu") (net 7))
 (segment (start 120 83.35) (end 120 78.64) (width 0.2) (layer "B.Cu") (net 7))
 (segment (start 125.21 97.63) (end 111.9 97.63) (width 0.2) (layer "B.Cu") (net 7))
 (segment (start 108.81 94.54) (end 120 83.35) (width 0.2) (layer "B.Cu") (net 7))
 (segment (start 119.38 49.11) (end 120.77 47.72) (width 0.2) (layer "B.Cu") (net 7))
 (segment (start 150.161314 97.63) (end 151.94 97.63) (width 0.2) (layer "B.Cu") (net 12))
 (segment (start 142.001057 32.709) (end 138.223057 36.487) (width 0.2) (layer "B.Cu") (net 12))
 (segment (start 144.37 97.63) (end 150.161314 97.63) (width 0.2) (layer "B.Cu") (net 12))
 (segment (start 152.81 93.22) (end 151.42 93.22) (width 0.2) (layer "B.Cu") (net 12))
 (segment (start 138.223057 36.487) (end 124.843 36.487) (width 0.2) (layer "B.Cu") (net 12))
 (segment (start 151.36 77.371314) (end 152.181 76.550314) (width 0.2) (layer "B.Cu") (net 12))
 (segment (start 153.4 93.81) (end 152.81 93.22) (width 0.2) (layer "B.Cu") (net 12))
 (segment (start 153.47 93.88) (end 153.4 93.81) (width 0.2) (layer "B.Cu") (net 12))
 (segment (start 155.91 46.1) (end 152.05 42.24) (width 0.2) (layer "B.Cu") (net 12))
 (segment (start 151.360314 93.210314) (end 151.36 93.21) (width 0.2) (layer "B.Cu") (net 12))
 (segment (start 142.498943 32.709) (end 142.001057 32.709) (width 0.2) (layer "B.Cu") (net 12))
 (segment (start 151.94 97.63) (end 153.47 96.1) (width 0.2) (layer "B.Cu") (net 12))
 (segment (start 155.91 67.25) (end 155.91 46.1) (width 0.2) (layer "B.Cu") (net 12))
 (segment (start 151.36 93.21) (end 151.36 77.371314) (width 0.2) (layer "B.Cu") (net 12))
 (segment (start 152.131 42.341057) (end 142.498943 32.709) (width 0.2) (layer "B.Cu") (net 12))
 (segment (start 152.181 76.550314) (end 152.181 75.389686) (width 0.2) (layer "B.Cu") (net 12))
 (segment (start 152.181 75.389686) (end 151.571 74.779686) (width 0.2) (layer "B.Cu") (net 12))
 (segment (start 151.571 71.589) (end 155.91 67.25) (width 0.2) (layer "B.Cu") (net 12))
 (segment (start 151.571 74.779686) (end 151.571 71.589) (width 0.2) (layer "B.Cu") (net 12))
 (segment (start 124.843 36.487) (end 121.08 40.25) (width 0.2) (layer "B.Cu") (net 12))
 (segment (start 153.47 96.1) (end 153.47 93.88) (width 0.2) (layer "B.Cu") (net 12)))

